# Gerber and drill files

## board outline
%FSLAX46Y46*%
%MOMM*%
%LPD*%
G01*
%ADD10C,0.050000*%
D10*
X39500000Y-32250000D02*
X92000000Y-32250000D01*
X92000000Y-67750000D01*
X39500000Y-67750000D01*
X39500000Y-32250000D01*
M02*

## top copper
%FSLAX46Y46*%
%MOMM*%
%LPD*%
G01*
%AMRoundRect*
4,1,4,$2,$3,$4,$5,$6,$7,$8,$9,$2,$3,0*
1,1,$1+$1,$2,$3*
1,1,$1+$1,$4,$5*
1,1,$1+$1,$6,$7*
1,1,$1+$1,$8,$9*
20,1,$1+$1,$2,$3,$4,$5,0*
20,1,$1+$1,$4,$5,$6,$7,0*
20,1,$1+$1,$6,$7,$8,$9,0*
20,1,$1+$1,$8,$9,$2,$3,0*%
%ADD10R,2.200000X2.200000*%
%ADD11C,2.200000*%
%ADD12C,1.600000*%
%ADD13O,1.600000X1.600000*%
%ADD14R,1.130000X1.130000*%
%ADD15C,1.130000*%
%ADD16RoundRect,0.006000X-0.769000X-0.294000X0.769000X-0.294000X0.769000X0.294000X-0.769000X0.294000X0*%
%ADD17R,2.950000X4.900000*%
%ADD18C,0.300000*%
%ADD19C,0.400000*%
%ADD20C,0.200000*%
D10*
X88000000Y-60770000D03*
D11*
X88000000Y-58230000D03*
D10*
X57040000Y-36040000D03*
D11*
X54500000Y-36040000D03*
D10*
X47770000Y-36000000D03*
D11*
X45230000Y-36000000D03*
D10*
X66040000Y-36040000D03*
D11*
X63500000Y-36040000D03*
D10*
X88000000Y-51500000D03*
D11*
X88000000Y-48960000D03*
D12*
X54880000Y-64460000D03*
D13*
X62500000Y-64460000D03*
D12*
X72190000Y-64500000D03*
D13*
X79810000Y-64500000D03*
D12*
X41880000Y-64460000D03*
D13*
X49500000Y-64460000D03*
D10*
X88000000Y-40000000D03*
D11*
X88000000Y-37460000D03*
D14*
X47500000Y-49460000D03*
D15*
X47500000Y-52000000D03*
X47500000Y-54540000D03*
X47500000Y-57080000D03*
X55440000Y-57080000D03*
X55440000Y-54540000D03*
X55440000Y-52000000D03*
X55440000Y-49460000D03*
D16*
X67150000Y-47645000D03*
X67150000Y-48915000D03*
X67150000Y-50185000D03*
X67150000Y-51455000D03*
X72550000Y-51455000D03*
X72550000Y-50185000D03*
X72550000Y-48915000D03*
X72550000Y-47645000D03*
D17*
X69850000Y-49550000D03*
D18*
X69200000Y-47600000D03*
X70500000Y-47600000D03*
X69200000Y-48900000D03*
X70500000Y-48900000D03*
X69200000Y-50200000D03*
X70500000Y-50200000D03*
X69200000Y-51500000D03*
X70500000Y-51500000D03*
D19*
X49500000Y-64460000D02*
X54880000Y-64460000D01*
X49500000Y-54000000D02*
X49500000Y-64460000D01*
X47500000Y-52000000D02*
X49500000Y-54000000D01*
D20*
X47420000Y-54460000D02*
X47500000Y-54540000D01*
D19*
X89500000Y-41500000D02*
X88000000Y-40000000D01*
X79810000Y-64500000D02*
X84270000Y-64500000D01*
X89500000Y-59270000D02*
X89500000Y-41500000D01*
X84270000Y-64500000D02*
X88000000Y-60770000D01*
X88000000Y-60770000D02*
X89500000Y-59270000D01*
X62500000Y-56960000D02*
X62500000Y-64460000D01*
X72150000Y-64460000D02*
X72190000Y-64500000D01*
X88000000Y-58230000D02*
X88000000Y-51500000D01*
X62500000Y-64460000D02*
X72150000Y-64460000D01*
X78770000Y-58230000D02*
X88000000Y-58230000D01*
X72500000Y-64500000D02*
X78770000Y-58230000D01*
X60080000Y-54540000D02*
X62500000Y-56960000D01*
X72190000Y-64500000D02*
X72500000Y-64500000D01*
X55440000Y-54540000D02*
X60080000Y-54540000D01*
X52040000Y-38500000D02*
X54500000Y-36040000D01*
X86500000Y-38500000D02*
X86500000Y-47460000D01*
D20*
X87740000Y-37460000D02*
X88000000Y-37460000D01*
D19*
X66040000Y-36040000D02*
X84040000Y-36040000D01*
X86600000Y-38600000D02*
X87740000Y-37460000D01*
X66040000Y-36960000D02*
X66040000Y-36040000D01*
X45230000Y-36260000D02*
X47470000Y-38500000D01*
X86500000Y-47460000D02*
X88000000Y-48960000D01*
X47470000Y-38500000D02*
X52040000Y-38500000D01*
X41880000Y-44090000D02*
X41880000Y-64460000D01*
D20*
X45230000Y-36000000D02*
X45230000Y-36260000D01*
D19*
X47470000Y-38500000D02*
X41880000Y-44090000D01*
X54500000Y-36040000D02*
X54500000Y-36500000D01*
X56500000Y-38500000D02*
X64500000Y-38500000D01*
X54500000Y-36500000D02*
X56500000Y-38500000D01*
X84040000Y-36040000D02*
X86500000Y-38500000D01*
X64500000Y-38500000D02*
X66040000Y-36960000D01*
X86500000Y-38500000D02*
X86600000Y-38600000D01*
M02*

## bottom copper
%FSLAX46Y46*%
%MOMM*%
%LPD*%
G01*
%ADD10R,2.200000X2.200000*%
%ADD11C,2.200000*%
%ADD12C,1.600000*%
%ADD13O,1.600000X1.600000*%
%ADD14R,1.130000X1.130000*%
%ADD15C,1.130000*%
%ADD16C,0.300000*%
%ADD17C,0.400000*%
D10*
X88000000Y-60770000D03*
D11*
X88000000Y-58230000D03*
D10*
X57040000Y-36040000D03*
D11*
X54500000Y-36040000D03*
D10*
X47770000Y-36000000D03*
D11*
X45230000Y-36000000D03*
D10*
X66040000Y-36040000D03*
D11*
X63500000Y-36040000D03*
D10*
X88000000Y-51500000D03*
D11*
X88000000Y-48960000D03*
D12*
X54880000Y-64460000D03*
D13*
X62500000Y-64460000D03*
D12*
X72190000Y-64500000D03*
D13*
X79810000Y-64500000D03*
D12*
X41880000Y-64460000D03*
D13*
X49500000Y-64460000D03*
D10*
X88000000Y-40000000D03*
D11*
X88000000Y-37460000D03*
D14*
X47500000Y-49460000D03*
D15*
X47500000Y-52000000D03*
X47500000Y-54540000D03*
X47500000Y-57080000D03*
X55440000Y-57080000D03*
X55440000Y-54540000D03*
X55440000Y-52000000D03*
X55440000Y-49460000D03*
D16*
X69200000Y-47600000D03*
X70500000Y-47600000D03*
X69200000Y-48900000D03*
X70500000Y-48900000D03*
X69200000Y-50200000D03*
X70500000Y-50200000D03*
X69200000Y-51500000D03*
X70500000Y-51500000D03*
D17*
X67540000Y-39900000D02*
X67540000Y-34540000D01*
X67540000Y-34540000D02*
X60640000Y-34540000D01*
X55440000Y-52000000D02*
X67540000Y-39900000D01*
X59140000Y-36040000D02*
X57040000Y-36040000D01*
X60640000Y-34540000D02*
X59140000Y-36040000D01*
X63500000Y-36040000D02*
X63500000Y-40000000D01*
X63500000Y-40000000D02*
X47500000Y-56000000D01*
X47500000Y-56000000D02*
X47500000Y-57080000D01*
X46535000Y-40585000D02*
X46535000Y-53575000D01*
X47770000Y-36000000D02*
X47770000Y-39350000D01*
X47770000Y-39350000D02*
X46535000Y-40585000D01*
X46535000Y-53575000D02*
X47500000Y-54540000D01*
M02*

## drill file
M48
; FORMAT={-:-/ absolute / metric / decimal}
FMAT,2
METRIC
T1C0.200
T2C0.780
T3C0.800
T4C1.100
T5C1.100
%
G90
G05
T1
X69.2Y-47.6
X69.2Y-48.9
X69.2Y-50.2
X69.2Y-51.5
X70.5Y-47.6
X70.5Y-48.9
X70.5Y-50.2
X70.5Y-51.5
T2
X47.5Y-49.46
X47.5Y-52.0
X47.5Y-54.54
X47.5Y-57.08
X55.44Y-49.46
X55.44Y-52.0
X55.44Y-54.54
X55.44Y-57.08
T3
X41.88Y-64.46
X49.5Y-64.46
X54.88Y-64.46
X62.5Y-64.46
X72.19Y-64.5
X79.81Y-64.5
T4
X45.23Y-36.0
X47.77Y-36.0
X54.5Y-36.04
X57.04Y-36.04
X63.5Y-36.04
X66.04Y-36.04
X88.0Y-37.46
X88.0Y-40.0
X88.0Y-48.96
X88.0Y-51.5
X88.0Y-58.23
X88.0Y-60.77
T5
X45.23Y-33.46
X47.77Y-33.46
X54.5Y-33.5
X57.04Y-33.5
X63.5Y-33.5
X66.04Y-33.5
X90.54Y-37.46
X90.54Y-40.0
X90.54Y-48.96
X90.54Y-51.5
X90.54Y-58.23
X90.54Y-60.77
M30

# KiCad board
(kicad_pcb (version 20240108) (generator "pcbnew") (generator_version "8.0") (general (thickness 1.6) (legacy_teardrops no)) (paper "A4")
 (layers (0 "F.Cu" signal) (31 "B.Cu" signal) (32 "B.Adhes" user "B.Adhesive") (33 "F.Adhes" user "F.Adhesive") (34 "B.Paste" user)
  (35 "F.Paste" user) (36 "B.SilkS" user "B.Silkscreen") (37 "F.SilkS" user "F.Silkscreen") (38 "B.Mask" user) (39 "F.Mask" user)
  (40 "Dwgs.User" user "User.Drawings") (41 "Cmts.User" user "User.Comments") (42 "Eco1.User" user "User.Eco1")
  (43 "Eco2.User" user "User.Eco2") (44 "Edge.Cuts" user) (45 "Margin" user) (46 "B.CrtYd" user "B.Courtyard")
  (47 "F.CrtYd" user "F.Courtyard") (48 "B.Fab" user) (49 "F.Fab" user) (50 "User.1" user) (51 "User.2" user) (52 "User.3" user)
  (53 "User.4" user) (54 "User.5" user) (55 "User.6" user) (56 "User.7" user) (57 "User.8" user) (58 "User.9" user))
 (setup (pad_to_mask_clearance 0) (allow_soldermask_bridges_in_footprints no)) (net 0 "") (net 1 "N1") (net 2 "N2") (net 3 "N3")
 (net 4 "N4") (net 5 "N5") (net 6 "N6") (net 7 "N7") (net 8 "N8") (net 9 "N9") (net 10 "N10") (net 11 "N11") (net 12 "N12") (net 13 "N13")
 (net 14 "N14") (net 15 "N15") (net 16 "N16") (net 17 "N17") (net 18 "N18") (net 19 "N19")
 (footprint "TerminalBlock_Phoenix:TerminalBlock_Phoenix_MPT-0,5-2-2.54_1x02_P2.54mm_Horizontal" (layer "F.Cu") (at 88 60.77 90)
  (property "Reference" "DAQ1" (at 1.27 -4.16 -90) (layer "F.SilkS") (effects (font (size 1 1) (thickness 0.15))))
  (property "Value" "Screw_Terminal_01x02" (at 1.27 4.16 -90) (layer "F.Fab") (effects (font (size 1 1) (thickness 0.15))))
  (pad "" np_thru_hole circle (at 0 2.54 90) (size 1.1 1.1) (drill 1.1) (layers "*.Cu" "*.Mask"))
  (pad "" np_thru_hole circle (at 2.54 2.54 90) (size 1.1 1.1) (drill 1.1) (layers "*.Cu" "*.Mask"))
  (pad "1" thru_hole rect (at 0 0 90) (size 2.2 2.2) (drill 1.1) (layers "*.Cu" "*.Mask") (remove_unused_layers no) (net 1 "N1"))
  (pad "2" thru_hole circle (at 2.54 0 90) (size 2.2 2.2) (drill 1.1) (layers "*.Cu" "*.Mask") (remove_unused_layers no) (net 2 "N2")))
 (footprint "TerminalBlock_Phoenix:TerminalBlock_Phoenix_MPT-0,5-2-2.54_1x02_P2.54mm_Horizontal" (layer "F.Cu") (at 57.04 36.04 180)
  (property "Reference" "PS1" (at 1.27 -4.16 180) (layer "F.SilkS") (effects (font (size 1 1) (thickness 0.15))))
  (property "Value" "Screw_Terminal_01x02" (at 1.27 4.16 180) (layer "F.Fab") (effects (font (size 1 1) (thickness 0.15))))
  (pad "" np_thru_hole circle (at 0 2.54 180) (size 1.1 1.1) (drill 1.1) (layers "*.Cu" "*.Mask"))
  (pad "" np_thru_hole circle (at 2.54 2.54 180) (size 1.1 1.1) (drill 1.1) (layers "*.Cu" "*.Mask"))
  (pad "1" thru_hole rect (at 0 0 180) (size 2.2 2.2) (drill 1.1) (layers "*.Cu" "*.Mask") (remove_unused_layers no) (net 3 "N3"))
  (pad "2" thru_hole circle (at 2.54 0 180) (size 2.2 2.2) (drill 1.1) (layers "*.Cu" "*.Mask") (remove_unused_layers no) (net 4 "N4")))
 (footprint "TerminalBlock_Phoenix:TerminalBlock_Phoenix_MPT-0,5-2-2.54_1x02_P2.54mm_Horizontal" (layer "F.Cu") (at 47.77 36 180)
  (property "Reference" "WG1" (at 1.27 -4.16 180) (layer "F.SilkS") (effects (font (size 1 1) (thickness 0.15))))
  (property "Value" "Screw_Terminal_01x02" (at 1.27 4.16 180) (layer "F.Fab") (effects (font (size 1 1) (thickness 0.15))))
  (pad "" np_thru_hole circle (at 0 2.54 180) (size 1.1 1.1) (drill 1.1) (layers "*.Cu" "*.Mask"))
  (pad "" np_thru_hole circle (at 2.54 2.54 180) (size 1.1 1.1) (drill 1.1) (layers "*.Cu" "*.Mask"))
  (pad "1" thru_hole rect (at 0 0 180) (size 2.2 2.2) (drill 1.1) (layers "*.Cu" "*.Mask") (remove_unused_layers no) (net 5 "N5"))
  (pad "2" thru_hole circle (at 2.54 0 180) (size 2.2 2.2) (drill 1.1) (layers "*.Cu" "*.Mask") (remove_unused_layers no) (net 4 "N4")))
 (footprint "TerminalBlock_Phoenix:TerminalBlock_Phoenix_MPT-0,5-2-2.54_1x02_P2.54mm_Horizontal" (layer "F.Cu") (at 66.04 36.04 180)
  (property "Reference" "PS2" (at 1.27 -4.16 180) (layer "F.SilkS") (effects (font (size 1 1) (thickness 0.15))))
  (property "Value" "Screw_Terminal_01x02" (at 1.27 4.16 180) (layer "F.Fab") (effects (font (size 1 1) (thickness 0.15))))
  (pad "" np_thru_hole circle (at 0 2.54 180) (size 1.1 1.1) (drill 1.1) (layers "*.Cu" "*.Mask"))
  (pad "" np_thru_hole circle (at 2.54 2.54 180) (size 1.1 1.1) (drill 1.1) (layers "*.Cu" "*.Mask"))
  (pad "1" thru_hole rect (at 0 0 180) (size 2.2 2.2) (drill 1.1) (layers "*.Cu" "*.Mask") (remove_unused_layers no) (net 4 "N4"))
  (pad "2" thru_hole circle (at 2.54 0 180) (size 2.2 2.2) (drill 1.1) (layers "*.Cu" "*.Mask") (remove_unused_layers no) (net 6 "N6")))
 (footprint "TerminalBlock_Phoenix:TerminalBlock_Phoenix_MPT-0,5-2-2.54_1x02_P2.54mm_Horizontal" (layer "F.Cu") (at 88 51.5 90)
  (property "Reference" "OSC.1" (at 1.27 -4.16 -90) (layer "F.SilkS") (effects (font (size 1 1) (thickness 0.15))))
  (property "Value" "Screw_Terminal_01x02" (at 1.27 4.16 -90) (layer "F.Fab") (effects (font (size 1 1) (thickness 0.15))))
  (pad "" np_thru_hole circle (at 0 2.54 90) (size 1.1 1.1) (drill 1.1) (layers "*.Cu" "*.Mask"))
  (pad "" np_thru_hole circle (at 2.54 2.54 90) (size 1.1 1.1) (drill 1.1) (layers "*.Cu" "*.Mask"))
  (pad "1" thru_hole rect (at 0 0 90) (size 2.2 2.2) (drill 1.1) (layers "*.Cu" "*.Mask") (remove_unused_layers no) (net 2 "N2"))
  (pad "2" thru_hole circle (at 2.54 0 90) (size 2.2 2.2) (drill 1.1) (layers "*.Cu" "*.Mask") (remove_unused_layers no) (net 4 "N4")))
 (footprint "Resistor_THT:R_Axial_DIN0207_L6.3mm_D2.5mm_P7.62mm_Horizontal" (layer "F.Cu") (at 54.88 64.46)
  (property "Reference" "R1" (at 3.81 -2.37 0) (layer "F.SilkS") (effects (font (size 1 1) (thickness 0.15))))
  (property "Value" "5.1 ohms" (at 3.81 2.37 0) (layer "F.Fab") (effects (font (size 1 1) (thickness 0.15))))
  (pad "1" thru_hole circle (at 0 0) (size 1.6 1.6) (drill 0.8) (layers "*.Cu" "*.Mask") (remove_unused_layers no) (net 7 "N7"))
  (pad "2" thru_hole oval (at 7.62 0) (size 1.6 1.6) (drill 0.8) (layers "*.Cu" "*.Mask") (remove_unused_layers no) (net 2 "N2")))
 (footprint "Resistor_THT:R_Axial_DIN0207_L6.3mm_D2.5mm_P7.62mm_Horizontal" (layer "F.Cu") (at 72.19 64.5)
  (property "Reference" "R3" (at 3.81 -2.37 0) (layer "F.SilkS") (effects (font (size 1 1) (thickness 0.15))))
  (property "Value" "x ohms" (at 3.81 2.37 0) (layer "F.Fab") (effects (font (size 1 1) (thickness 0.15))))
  (pad "1" thru_hole circle (at 0 0) (size 1.6 1.6) (drill 0.8) (layers "*.Cu" "*.Mask") (remove_unused_layers no) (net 2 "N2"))
  (pad "2" thru_hole oval (at 7.62 0) (size 1.6 1.6) (drill 0.8) (layers "*.Cu" "*.Mask") (remove_unused_layers no) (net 1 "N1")))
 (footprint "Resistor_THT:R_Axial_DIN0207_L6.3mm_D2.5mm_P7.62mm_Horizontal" (layer "F.Cu") (at 41.88 64.46)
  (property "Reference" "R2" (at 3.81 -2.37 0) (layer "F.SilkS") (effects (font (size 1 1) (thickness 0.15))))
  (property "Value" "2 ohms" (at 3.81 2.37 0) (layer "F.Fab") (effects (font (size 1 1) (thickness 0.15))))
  (pad "1" thru_hole circle (at 0 0) (size 1.6 1.6) (drill 0.8) (layers "*.Cu" "*.Mask") (remove_unused_layers no) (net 4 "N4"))
  (pad "2" thru_hole oval (at 7.62 0) (size 1.6 1.6) (drill 0.8) (layers "*.Cu" "*.Mask") (remove_unused_layers no) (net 7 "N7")))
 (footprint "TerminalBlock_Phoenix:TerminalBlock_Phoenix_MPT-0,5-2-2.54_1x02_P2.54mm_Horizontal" (layer "F.Cu") (at 88 40 90)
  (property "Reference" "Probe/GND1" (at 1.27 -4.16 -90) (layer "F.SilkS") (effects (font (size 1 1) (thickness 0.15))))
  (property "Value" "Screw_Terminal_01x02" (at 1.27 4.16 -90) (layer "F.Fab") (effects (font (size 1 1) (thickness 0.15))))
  (pad "" np_thru_hole circle (at 0 2.54 90) (size 1.1 1.1) (drill 1.1) (layers "*.Cu" "*.Mask"))
  (pad "" np_thru_hole circle (at 2.54 2.54 90) (size 1.1 1.1) (drill 1.1) (layers "*.Cu" "*.Mask"))
  (pad "1" thru_hole rect (at 0 0 90) (size 2.2 2.2) (drill 1.1) (layers "*.Cu" "*.Mask") (remove_unused_layers no) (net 1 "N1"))
  (pad "2" thru_hole circle (at 2.54 0 90) (size 2.2 2.2) (drill 1.1) (layers "*.Cu" "*.Mask") (remove_unused_layers no) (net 4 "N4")))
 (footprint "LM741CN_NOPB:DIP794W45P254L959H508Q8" (layer "F.Cu") (at 51.47 53.27)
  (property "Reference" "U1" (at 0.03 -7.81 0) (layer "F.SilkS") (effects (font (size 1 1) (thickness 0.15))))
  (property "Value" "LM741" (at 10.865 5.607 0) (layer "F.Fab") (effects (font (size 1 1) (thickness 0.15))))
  (pad "1" thru_hole rect (at -3.97 -3.81) (size 1.13 1.13) (drill 0.78) (layers "*.Cu" "*.Mask") (remove_unused_layers no) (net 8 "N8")
   (solder_mask_margin 0.102))
  (pad "2" thru_hole circle (at -3.97 -1.27) (size 1.13 1.13) (drill 0.78) (layers "*.Cu" "*.Mask") (remove_unused_layers no) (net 7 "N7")
   (solder_mask_margin 0.102))
  (pad "3" thru_hole circle (at -3.97 1.27) (size 1.13 1.13) (drill 0.78) (layers "*.Cu" "*.Mask") (remove_unused_layers no) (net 5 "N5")
   (solder_mask_margin 0.102))
  (pad "4" thru_hole circle (at -3.97 3.81) (size 1.13 1.13) (drill 0.78) (layers "*.Cu" "*.Mask") (remove_unused_layers no) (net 6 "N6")
   (solder_mask_margin 0.102))
  (pad "5" thru_hole circle (at 3.97 3.81) (size 1.13 1.13) (drill 0.78) (layers "*.Cu" "*.Mask") (remove_unused_layers no) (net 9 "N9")
   (solder_mask_margin 0.102))
  (pad "6" thru_hole circle (at 3.97 1.27) (size 1.13 1.13) (drill 0.78) (layers "*.Cu" "*.Mask") (remove_unused_layers no) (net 2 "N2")
   (solder_mask_margin 0.102))
  (pad "7" thru_hole circle (at 3.97 -1.27) (size 1.13 1.13) (drill 0.78) (layers "*.Cu" "*.Mask") (remove_unused_layers no) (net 3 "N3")
   (solder_mask_margin 0.102))
  (pad "8" thru_hole circle (at 3.97 -3.81) (size 1.13 1.13) (drill 0.78) (layers "*.Cu" "*.Mask") (remove_unused_layers no) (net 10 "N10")
   (solder_mask_margin 0.102)))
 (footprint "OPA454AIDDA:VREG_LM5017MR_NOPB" (layer "F.Cu") (at 69.85 49.55)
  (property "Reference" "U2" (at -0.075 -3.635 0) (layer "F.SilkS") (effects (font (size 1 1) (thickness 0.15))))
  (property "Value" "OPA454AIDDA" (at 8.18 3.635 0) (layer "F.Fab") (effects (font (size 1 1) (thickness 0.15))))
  (pad "1" smd roundrect (at -2.7 -1.905) (size 1.55 0.6) (layers "F.Cu" "F.Paste") (roundrect_rratio 0.01) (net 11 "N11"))
  (pad "2" smd roundrect (at -2.7 -0.635) (size 1.55 0.6) (layers "F.Cu" "F.Paste") (roundrect_rratio 0.01) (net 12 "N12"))
  (pad "3" smd roundrect (at -2.7 0.635) (size 1.55 0.6) (layers "F.Cu" "F.Paste") (roundrect_rratio 0.01) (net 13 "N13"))
  (pad "4" smd roundrect (at -2.7 1.905) (size 1.55 0.6) (layers "F.Cu" "F.Paste") (roundrect_rratio 0.01) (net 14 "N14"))
  (pad "5" smd roundrect (at 2.7 1.905) (size 1.55 0.6) (layers "F.Cu" "F.Paste") (roundrect_rratio 0.01) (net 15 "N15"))
  (pad "6" smd roundrect (at 2.7 0.635) (size 1.55 0.6) (layers "F.Cu" "F.Paste") (roundrect_rratio 0.01) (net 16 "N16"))
  (pad "7" smd roundrect (at 2.7 -0.635) (size 1.55 0.6) (layers "F.Cu" "F.Paste") (roundrect_rratio 0.01) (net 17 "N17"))
  (pad "8" smd roundrect (at 2.7 -1.905) (size 1.55 0.6) (layers "F.Cu" "F.Paste") (roundrect_rratio 0.01) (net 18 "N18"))
  (pad "9" smd rect (at 0 0) (size 2.95 4.9) (layers "F.Cu") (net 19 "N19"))
  (pad "10" thru_hole circle (at -0.65 -1.95) (size 0.3 0.3) (drill 0.2) (layers "*.Cu" "*.Mask") (remove_unused_layers no)
   (solder_mask_margin 0.102))
  (pad "11" thru_hole circle (at 0.65 -1.95) (size 0.3 0.3) (drill 0.2) (layers "*.Cu" "*.Mask") (remove_unused_layers no)
   (solder_mask_margin 0.102))
  (pad "12" thru_hole circle (at -0.65 -0.65) (size 0.3 0.3) (drill 0.2) (layers "*.Cu" "*.Mask") (remove_unused_layers no)
   (solder_mask_margin 0.102))
  (pad "13" thru_hole circle (at 0.65 -0.65) (size 0.3 0.3) (drill 0.2) (layers "*.Cu" "*.Mask") (remove_unused_layers no)
   (solder_mask_margin 0.102))
  (pad "14" thru_hole circle (at -0.65 0.65) (size 0.3 0.3) (drill 0.2) (layers "*.Cu" "*.Mask") (remove_unused_layers no)
   (solder_mask_margin 0.102))
  (pad "15" thru_hole circle (at 0.65 0.65) (size 0.3 0.3) (drill 0.2) (layers "*.Cu" "*.Mask") (remove_unused_layers no)
   (solder_mask_margin 0.102))
  (pad "16" thru_hole circle (at -0.65 1.95) (size 0.3 0.3) (drill 0.2) (layers "*.Cu" "*.Mask") (remove_unused_layers no)
   (solder_mask_margin 0.102))
  (pad "17" thru_hole circle (at 0.65 1.95) (size 0.3 0.3) (drill 0.2) (layers "*.Cu" "*.Mask") (remove_unused_layers no)
   (solder_mask_margin 0.102)))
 (gr_rect (start 39.5 32.25) (end 92 67.75) (stroke (width 0.05) (type default)) (fill none) (layer "Edge.Cuts"))
 (segment (start 49.5 64.46) (end 54.88 64.46) (width 0.4) (layer "F.Cu") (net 7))
 (segment (start 49.5 54) (end 49.5 64.46) (width 0.4) (layer "F.Cu") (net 7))
 (segment (start 47.5 52) (end 49.5 54) (width 0.4) (layer "F.Cu") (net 7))
 (segment (start 67.54 39.9) (end 67.54 34.54) (width 0.4) (layer "B.Cu") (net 3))
 (segment (start 67.54 34.54) (end 60.64 34.54) (width 0.4) (layer "B.Cu") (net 3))
 (segment (start 55.44 52) (end 67.54 39.9) (width 0.4) (layer "B.Cu") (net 3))
 (segment (start 59.14 36.04) (end 57.04 36.04) (width 0.4) (layer "B.Cu") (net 3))
 (segment (start 60.64 34.54) (end 59.14 36.04) (width 0.4) (layer "B.Cu") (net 3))
 (segment (start 63.5 36.04) (end 63.5 40) (width 0.4) (layer "B.Cu") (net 6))
 (segment (start 63.5 40) (end 47.5 56) (width 0.4) (layer "B.Cu") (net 6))
 (segment (start 47.5 56) (end 47.5 57.08) (width 0.4) (layer "B.Cu") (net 6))
 (segment (start 47.42 54.46) (end 47.5 54.54) (width 0.2) (layer "F.Cu") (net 5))
 (segment (start 46.535 40.585) (end 46.535 53.575) (width 0.4) (layer "B.Cu") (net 5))
 (segment (start 47.77 36) (end 47.77 39.35) (width 0.4) (layer "B.Cu") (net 5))
 (segment (start 47.77 39.35) (end 46.535 40.585) (width 0.4) (layer "B.Cu") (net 5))
 (segment (start 46.535 53.575) (end 47.5 54.54) (width 0.4) (layer "B.Cu") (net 5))
 (segment (start 89.5 41.5) (end 88 40) (width 0.4) (layer "F.Cu") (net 1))
 (segment (start 79.81 64.5) (end 84.27 64.5) (width 0.4) (layer "F.Cu") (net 1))
 (segment (start 89.5 59.27) (end 89.5 41.5) (width 0.4) (layer "F.Cu") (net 1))
 (segment (start 84.27 64.5) (end 88 60.77) (width 0.4) (layer "F.Cu") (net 1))
 (segment (start 88 60.77) (end 89.5 59.27) (width 0.4) (layer "F.Cu") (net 1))
 (segment (start 62.5 56.96) (end 62.5 64.46) (width 0.4) (layer "F.Cu") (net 2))
 (segment (start 72.15 64.46) (end 72.19 64.5) (width 0.4) (layer "F.Cu") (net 2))
 (segment (start 88 58.23) (end 88 51.5) (width 0.4) (layer "F.Cu") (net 2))
 (segment (start 62.5 64.46) (end 72.15 64.46) (width 0.4) (layer "F.Cu") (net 2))
 (segment (start 78.77 58.23) (end 88 58.23) (width 0.4) (layer "F.Cu") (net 2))
 (segment (start 72.5 64.5) (end 78.77 58.23) (width 0.4) (layer "F.Cu") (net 2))
 (segment (start 60.08 54.54) (end 62.5 56.96) (width 0.4) (layer "F.Cu") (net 2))
 (segment (start 72.19 64.5) (end 72.5 64.5) (width 0.4) (layer "F.Cu") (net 2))
 (segment (start 55.44 54.54) (end 60.08 54.54) (width 0.4) (layer "F.Cu") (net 2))
 (segment (start 52.04 38.5) (end 54.5 36.04) (width 0.4) (layer "F.Cu") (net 4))
 (segment (start 86.5 38.5) (end 86.5 47.46) (width 0.4) (layer "F.Cu") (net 4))
 (segment (start 87.74 37.46) (end 88 37.46) (width 0.2) (layer "F.Cu") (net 4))
 (segment (start 66.04 36.04) (end 84.04 36.04) (width 0.4) (layer "F.Cu") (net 4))
 (segment (start 86.6 38.6) (end 87.74 37.46) (width 0.4) (layer "F.Cu") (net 4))
 (segment (start 66.04 36.96) (end 66.04 36.04) (width 0.4) (layer "F.Cu") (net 4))
 (segment (start 45.23 36.26) (end 47.47 38.5) (width 0.4) (layer "F.Cu") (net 4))
 (segment (start 86.5 47.46) (end 88 48.96) (width 0.4) (layer "F.Cu") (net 4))
 (segment (start 47.47 38.5) (end 52.04 38.5) (width 0.4) (layer "F.Cu") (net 4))
 (segment (start 41.88 44.09) (end 41.88 64.46) (width 0.4) (layer "F.Cu") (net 4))
 (segment (start 45.23 36) (end 45.23 36.26) (width 0.2) (layer "F.Cu") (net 4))
 (segment (start 47.47 38.5) (end 41.88 44.09) (width 0.4) (layer "F.Cu") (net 4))
 (segment (start 54.5 36.04) (end 54.5 36.5) (width 0.4) (layer "F.Cu") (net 4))
 (segment (start 56.5 38.5) (end 64.5 38.5) (width 0.4) (layer "F.Cu") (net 4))
 (segment (start 54.5 36.5) (end 56.5 38.5) (width 0.4) (layer "F.Cu") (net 4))
 (segment (start 84.04 36.04) (end 86.5 38.5) (width 0.4) (layer "F.Cu") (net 4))
 (segment (start 64.5 38.5) (end 66.04 36.96) (width 0.4) (layer "F.Cu") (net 4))
 (segment (start 86.5 38.5) (end 86.6 38.6) (width 0.4) (layer "F.Cu") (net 4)))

